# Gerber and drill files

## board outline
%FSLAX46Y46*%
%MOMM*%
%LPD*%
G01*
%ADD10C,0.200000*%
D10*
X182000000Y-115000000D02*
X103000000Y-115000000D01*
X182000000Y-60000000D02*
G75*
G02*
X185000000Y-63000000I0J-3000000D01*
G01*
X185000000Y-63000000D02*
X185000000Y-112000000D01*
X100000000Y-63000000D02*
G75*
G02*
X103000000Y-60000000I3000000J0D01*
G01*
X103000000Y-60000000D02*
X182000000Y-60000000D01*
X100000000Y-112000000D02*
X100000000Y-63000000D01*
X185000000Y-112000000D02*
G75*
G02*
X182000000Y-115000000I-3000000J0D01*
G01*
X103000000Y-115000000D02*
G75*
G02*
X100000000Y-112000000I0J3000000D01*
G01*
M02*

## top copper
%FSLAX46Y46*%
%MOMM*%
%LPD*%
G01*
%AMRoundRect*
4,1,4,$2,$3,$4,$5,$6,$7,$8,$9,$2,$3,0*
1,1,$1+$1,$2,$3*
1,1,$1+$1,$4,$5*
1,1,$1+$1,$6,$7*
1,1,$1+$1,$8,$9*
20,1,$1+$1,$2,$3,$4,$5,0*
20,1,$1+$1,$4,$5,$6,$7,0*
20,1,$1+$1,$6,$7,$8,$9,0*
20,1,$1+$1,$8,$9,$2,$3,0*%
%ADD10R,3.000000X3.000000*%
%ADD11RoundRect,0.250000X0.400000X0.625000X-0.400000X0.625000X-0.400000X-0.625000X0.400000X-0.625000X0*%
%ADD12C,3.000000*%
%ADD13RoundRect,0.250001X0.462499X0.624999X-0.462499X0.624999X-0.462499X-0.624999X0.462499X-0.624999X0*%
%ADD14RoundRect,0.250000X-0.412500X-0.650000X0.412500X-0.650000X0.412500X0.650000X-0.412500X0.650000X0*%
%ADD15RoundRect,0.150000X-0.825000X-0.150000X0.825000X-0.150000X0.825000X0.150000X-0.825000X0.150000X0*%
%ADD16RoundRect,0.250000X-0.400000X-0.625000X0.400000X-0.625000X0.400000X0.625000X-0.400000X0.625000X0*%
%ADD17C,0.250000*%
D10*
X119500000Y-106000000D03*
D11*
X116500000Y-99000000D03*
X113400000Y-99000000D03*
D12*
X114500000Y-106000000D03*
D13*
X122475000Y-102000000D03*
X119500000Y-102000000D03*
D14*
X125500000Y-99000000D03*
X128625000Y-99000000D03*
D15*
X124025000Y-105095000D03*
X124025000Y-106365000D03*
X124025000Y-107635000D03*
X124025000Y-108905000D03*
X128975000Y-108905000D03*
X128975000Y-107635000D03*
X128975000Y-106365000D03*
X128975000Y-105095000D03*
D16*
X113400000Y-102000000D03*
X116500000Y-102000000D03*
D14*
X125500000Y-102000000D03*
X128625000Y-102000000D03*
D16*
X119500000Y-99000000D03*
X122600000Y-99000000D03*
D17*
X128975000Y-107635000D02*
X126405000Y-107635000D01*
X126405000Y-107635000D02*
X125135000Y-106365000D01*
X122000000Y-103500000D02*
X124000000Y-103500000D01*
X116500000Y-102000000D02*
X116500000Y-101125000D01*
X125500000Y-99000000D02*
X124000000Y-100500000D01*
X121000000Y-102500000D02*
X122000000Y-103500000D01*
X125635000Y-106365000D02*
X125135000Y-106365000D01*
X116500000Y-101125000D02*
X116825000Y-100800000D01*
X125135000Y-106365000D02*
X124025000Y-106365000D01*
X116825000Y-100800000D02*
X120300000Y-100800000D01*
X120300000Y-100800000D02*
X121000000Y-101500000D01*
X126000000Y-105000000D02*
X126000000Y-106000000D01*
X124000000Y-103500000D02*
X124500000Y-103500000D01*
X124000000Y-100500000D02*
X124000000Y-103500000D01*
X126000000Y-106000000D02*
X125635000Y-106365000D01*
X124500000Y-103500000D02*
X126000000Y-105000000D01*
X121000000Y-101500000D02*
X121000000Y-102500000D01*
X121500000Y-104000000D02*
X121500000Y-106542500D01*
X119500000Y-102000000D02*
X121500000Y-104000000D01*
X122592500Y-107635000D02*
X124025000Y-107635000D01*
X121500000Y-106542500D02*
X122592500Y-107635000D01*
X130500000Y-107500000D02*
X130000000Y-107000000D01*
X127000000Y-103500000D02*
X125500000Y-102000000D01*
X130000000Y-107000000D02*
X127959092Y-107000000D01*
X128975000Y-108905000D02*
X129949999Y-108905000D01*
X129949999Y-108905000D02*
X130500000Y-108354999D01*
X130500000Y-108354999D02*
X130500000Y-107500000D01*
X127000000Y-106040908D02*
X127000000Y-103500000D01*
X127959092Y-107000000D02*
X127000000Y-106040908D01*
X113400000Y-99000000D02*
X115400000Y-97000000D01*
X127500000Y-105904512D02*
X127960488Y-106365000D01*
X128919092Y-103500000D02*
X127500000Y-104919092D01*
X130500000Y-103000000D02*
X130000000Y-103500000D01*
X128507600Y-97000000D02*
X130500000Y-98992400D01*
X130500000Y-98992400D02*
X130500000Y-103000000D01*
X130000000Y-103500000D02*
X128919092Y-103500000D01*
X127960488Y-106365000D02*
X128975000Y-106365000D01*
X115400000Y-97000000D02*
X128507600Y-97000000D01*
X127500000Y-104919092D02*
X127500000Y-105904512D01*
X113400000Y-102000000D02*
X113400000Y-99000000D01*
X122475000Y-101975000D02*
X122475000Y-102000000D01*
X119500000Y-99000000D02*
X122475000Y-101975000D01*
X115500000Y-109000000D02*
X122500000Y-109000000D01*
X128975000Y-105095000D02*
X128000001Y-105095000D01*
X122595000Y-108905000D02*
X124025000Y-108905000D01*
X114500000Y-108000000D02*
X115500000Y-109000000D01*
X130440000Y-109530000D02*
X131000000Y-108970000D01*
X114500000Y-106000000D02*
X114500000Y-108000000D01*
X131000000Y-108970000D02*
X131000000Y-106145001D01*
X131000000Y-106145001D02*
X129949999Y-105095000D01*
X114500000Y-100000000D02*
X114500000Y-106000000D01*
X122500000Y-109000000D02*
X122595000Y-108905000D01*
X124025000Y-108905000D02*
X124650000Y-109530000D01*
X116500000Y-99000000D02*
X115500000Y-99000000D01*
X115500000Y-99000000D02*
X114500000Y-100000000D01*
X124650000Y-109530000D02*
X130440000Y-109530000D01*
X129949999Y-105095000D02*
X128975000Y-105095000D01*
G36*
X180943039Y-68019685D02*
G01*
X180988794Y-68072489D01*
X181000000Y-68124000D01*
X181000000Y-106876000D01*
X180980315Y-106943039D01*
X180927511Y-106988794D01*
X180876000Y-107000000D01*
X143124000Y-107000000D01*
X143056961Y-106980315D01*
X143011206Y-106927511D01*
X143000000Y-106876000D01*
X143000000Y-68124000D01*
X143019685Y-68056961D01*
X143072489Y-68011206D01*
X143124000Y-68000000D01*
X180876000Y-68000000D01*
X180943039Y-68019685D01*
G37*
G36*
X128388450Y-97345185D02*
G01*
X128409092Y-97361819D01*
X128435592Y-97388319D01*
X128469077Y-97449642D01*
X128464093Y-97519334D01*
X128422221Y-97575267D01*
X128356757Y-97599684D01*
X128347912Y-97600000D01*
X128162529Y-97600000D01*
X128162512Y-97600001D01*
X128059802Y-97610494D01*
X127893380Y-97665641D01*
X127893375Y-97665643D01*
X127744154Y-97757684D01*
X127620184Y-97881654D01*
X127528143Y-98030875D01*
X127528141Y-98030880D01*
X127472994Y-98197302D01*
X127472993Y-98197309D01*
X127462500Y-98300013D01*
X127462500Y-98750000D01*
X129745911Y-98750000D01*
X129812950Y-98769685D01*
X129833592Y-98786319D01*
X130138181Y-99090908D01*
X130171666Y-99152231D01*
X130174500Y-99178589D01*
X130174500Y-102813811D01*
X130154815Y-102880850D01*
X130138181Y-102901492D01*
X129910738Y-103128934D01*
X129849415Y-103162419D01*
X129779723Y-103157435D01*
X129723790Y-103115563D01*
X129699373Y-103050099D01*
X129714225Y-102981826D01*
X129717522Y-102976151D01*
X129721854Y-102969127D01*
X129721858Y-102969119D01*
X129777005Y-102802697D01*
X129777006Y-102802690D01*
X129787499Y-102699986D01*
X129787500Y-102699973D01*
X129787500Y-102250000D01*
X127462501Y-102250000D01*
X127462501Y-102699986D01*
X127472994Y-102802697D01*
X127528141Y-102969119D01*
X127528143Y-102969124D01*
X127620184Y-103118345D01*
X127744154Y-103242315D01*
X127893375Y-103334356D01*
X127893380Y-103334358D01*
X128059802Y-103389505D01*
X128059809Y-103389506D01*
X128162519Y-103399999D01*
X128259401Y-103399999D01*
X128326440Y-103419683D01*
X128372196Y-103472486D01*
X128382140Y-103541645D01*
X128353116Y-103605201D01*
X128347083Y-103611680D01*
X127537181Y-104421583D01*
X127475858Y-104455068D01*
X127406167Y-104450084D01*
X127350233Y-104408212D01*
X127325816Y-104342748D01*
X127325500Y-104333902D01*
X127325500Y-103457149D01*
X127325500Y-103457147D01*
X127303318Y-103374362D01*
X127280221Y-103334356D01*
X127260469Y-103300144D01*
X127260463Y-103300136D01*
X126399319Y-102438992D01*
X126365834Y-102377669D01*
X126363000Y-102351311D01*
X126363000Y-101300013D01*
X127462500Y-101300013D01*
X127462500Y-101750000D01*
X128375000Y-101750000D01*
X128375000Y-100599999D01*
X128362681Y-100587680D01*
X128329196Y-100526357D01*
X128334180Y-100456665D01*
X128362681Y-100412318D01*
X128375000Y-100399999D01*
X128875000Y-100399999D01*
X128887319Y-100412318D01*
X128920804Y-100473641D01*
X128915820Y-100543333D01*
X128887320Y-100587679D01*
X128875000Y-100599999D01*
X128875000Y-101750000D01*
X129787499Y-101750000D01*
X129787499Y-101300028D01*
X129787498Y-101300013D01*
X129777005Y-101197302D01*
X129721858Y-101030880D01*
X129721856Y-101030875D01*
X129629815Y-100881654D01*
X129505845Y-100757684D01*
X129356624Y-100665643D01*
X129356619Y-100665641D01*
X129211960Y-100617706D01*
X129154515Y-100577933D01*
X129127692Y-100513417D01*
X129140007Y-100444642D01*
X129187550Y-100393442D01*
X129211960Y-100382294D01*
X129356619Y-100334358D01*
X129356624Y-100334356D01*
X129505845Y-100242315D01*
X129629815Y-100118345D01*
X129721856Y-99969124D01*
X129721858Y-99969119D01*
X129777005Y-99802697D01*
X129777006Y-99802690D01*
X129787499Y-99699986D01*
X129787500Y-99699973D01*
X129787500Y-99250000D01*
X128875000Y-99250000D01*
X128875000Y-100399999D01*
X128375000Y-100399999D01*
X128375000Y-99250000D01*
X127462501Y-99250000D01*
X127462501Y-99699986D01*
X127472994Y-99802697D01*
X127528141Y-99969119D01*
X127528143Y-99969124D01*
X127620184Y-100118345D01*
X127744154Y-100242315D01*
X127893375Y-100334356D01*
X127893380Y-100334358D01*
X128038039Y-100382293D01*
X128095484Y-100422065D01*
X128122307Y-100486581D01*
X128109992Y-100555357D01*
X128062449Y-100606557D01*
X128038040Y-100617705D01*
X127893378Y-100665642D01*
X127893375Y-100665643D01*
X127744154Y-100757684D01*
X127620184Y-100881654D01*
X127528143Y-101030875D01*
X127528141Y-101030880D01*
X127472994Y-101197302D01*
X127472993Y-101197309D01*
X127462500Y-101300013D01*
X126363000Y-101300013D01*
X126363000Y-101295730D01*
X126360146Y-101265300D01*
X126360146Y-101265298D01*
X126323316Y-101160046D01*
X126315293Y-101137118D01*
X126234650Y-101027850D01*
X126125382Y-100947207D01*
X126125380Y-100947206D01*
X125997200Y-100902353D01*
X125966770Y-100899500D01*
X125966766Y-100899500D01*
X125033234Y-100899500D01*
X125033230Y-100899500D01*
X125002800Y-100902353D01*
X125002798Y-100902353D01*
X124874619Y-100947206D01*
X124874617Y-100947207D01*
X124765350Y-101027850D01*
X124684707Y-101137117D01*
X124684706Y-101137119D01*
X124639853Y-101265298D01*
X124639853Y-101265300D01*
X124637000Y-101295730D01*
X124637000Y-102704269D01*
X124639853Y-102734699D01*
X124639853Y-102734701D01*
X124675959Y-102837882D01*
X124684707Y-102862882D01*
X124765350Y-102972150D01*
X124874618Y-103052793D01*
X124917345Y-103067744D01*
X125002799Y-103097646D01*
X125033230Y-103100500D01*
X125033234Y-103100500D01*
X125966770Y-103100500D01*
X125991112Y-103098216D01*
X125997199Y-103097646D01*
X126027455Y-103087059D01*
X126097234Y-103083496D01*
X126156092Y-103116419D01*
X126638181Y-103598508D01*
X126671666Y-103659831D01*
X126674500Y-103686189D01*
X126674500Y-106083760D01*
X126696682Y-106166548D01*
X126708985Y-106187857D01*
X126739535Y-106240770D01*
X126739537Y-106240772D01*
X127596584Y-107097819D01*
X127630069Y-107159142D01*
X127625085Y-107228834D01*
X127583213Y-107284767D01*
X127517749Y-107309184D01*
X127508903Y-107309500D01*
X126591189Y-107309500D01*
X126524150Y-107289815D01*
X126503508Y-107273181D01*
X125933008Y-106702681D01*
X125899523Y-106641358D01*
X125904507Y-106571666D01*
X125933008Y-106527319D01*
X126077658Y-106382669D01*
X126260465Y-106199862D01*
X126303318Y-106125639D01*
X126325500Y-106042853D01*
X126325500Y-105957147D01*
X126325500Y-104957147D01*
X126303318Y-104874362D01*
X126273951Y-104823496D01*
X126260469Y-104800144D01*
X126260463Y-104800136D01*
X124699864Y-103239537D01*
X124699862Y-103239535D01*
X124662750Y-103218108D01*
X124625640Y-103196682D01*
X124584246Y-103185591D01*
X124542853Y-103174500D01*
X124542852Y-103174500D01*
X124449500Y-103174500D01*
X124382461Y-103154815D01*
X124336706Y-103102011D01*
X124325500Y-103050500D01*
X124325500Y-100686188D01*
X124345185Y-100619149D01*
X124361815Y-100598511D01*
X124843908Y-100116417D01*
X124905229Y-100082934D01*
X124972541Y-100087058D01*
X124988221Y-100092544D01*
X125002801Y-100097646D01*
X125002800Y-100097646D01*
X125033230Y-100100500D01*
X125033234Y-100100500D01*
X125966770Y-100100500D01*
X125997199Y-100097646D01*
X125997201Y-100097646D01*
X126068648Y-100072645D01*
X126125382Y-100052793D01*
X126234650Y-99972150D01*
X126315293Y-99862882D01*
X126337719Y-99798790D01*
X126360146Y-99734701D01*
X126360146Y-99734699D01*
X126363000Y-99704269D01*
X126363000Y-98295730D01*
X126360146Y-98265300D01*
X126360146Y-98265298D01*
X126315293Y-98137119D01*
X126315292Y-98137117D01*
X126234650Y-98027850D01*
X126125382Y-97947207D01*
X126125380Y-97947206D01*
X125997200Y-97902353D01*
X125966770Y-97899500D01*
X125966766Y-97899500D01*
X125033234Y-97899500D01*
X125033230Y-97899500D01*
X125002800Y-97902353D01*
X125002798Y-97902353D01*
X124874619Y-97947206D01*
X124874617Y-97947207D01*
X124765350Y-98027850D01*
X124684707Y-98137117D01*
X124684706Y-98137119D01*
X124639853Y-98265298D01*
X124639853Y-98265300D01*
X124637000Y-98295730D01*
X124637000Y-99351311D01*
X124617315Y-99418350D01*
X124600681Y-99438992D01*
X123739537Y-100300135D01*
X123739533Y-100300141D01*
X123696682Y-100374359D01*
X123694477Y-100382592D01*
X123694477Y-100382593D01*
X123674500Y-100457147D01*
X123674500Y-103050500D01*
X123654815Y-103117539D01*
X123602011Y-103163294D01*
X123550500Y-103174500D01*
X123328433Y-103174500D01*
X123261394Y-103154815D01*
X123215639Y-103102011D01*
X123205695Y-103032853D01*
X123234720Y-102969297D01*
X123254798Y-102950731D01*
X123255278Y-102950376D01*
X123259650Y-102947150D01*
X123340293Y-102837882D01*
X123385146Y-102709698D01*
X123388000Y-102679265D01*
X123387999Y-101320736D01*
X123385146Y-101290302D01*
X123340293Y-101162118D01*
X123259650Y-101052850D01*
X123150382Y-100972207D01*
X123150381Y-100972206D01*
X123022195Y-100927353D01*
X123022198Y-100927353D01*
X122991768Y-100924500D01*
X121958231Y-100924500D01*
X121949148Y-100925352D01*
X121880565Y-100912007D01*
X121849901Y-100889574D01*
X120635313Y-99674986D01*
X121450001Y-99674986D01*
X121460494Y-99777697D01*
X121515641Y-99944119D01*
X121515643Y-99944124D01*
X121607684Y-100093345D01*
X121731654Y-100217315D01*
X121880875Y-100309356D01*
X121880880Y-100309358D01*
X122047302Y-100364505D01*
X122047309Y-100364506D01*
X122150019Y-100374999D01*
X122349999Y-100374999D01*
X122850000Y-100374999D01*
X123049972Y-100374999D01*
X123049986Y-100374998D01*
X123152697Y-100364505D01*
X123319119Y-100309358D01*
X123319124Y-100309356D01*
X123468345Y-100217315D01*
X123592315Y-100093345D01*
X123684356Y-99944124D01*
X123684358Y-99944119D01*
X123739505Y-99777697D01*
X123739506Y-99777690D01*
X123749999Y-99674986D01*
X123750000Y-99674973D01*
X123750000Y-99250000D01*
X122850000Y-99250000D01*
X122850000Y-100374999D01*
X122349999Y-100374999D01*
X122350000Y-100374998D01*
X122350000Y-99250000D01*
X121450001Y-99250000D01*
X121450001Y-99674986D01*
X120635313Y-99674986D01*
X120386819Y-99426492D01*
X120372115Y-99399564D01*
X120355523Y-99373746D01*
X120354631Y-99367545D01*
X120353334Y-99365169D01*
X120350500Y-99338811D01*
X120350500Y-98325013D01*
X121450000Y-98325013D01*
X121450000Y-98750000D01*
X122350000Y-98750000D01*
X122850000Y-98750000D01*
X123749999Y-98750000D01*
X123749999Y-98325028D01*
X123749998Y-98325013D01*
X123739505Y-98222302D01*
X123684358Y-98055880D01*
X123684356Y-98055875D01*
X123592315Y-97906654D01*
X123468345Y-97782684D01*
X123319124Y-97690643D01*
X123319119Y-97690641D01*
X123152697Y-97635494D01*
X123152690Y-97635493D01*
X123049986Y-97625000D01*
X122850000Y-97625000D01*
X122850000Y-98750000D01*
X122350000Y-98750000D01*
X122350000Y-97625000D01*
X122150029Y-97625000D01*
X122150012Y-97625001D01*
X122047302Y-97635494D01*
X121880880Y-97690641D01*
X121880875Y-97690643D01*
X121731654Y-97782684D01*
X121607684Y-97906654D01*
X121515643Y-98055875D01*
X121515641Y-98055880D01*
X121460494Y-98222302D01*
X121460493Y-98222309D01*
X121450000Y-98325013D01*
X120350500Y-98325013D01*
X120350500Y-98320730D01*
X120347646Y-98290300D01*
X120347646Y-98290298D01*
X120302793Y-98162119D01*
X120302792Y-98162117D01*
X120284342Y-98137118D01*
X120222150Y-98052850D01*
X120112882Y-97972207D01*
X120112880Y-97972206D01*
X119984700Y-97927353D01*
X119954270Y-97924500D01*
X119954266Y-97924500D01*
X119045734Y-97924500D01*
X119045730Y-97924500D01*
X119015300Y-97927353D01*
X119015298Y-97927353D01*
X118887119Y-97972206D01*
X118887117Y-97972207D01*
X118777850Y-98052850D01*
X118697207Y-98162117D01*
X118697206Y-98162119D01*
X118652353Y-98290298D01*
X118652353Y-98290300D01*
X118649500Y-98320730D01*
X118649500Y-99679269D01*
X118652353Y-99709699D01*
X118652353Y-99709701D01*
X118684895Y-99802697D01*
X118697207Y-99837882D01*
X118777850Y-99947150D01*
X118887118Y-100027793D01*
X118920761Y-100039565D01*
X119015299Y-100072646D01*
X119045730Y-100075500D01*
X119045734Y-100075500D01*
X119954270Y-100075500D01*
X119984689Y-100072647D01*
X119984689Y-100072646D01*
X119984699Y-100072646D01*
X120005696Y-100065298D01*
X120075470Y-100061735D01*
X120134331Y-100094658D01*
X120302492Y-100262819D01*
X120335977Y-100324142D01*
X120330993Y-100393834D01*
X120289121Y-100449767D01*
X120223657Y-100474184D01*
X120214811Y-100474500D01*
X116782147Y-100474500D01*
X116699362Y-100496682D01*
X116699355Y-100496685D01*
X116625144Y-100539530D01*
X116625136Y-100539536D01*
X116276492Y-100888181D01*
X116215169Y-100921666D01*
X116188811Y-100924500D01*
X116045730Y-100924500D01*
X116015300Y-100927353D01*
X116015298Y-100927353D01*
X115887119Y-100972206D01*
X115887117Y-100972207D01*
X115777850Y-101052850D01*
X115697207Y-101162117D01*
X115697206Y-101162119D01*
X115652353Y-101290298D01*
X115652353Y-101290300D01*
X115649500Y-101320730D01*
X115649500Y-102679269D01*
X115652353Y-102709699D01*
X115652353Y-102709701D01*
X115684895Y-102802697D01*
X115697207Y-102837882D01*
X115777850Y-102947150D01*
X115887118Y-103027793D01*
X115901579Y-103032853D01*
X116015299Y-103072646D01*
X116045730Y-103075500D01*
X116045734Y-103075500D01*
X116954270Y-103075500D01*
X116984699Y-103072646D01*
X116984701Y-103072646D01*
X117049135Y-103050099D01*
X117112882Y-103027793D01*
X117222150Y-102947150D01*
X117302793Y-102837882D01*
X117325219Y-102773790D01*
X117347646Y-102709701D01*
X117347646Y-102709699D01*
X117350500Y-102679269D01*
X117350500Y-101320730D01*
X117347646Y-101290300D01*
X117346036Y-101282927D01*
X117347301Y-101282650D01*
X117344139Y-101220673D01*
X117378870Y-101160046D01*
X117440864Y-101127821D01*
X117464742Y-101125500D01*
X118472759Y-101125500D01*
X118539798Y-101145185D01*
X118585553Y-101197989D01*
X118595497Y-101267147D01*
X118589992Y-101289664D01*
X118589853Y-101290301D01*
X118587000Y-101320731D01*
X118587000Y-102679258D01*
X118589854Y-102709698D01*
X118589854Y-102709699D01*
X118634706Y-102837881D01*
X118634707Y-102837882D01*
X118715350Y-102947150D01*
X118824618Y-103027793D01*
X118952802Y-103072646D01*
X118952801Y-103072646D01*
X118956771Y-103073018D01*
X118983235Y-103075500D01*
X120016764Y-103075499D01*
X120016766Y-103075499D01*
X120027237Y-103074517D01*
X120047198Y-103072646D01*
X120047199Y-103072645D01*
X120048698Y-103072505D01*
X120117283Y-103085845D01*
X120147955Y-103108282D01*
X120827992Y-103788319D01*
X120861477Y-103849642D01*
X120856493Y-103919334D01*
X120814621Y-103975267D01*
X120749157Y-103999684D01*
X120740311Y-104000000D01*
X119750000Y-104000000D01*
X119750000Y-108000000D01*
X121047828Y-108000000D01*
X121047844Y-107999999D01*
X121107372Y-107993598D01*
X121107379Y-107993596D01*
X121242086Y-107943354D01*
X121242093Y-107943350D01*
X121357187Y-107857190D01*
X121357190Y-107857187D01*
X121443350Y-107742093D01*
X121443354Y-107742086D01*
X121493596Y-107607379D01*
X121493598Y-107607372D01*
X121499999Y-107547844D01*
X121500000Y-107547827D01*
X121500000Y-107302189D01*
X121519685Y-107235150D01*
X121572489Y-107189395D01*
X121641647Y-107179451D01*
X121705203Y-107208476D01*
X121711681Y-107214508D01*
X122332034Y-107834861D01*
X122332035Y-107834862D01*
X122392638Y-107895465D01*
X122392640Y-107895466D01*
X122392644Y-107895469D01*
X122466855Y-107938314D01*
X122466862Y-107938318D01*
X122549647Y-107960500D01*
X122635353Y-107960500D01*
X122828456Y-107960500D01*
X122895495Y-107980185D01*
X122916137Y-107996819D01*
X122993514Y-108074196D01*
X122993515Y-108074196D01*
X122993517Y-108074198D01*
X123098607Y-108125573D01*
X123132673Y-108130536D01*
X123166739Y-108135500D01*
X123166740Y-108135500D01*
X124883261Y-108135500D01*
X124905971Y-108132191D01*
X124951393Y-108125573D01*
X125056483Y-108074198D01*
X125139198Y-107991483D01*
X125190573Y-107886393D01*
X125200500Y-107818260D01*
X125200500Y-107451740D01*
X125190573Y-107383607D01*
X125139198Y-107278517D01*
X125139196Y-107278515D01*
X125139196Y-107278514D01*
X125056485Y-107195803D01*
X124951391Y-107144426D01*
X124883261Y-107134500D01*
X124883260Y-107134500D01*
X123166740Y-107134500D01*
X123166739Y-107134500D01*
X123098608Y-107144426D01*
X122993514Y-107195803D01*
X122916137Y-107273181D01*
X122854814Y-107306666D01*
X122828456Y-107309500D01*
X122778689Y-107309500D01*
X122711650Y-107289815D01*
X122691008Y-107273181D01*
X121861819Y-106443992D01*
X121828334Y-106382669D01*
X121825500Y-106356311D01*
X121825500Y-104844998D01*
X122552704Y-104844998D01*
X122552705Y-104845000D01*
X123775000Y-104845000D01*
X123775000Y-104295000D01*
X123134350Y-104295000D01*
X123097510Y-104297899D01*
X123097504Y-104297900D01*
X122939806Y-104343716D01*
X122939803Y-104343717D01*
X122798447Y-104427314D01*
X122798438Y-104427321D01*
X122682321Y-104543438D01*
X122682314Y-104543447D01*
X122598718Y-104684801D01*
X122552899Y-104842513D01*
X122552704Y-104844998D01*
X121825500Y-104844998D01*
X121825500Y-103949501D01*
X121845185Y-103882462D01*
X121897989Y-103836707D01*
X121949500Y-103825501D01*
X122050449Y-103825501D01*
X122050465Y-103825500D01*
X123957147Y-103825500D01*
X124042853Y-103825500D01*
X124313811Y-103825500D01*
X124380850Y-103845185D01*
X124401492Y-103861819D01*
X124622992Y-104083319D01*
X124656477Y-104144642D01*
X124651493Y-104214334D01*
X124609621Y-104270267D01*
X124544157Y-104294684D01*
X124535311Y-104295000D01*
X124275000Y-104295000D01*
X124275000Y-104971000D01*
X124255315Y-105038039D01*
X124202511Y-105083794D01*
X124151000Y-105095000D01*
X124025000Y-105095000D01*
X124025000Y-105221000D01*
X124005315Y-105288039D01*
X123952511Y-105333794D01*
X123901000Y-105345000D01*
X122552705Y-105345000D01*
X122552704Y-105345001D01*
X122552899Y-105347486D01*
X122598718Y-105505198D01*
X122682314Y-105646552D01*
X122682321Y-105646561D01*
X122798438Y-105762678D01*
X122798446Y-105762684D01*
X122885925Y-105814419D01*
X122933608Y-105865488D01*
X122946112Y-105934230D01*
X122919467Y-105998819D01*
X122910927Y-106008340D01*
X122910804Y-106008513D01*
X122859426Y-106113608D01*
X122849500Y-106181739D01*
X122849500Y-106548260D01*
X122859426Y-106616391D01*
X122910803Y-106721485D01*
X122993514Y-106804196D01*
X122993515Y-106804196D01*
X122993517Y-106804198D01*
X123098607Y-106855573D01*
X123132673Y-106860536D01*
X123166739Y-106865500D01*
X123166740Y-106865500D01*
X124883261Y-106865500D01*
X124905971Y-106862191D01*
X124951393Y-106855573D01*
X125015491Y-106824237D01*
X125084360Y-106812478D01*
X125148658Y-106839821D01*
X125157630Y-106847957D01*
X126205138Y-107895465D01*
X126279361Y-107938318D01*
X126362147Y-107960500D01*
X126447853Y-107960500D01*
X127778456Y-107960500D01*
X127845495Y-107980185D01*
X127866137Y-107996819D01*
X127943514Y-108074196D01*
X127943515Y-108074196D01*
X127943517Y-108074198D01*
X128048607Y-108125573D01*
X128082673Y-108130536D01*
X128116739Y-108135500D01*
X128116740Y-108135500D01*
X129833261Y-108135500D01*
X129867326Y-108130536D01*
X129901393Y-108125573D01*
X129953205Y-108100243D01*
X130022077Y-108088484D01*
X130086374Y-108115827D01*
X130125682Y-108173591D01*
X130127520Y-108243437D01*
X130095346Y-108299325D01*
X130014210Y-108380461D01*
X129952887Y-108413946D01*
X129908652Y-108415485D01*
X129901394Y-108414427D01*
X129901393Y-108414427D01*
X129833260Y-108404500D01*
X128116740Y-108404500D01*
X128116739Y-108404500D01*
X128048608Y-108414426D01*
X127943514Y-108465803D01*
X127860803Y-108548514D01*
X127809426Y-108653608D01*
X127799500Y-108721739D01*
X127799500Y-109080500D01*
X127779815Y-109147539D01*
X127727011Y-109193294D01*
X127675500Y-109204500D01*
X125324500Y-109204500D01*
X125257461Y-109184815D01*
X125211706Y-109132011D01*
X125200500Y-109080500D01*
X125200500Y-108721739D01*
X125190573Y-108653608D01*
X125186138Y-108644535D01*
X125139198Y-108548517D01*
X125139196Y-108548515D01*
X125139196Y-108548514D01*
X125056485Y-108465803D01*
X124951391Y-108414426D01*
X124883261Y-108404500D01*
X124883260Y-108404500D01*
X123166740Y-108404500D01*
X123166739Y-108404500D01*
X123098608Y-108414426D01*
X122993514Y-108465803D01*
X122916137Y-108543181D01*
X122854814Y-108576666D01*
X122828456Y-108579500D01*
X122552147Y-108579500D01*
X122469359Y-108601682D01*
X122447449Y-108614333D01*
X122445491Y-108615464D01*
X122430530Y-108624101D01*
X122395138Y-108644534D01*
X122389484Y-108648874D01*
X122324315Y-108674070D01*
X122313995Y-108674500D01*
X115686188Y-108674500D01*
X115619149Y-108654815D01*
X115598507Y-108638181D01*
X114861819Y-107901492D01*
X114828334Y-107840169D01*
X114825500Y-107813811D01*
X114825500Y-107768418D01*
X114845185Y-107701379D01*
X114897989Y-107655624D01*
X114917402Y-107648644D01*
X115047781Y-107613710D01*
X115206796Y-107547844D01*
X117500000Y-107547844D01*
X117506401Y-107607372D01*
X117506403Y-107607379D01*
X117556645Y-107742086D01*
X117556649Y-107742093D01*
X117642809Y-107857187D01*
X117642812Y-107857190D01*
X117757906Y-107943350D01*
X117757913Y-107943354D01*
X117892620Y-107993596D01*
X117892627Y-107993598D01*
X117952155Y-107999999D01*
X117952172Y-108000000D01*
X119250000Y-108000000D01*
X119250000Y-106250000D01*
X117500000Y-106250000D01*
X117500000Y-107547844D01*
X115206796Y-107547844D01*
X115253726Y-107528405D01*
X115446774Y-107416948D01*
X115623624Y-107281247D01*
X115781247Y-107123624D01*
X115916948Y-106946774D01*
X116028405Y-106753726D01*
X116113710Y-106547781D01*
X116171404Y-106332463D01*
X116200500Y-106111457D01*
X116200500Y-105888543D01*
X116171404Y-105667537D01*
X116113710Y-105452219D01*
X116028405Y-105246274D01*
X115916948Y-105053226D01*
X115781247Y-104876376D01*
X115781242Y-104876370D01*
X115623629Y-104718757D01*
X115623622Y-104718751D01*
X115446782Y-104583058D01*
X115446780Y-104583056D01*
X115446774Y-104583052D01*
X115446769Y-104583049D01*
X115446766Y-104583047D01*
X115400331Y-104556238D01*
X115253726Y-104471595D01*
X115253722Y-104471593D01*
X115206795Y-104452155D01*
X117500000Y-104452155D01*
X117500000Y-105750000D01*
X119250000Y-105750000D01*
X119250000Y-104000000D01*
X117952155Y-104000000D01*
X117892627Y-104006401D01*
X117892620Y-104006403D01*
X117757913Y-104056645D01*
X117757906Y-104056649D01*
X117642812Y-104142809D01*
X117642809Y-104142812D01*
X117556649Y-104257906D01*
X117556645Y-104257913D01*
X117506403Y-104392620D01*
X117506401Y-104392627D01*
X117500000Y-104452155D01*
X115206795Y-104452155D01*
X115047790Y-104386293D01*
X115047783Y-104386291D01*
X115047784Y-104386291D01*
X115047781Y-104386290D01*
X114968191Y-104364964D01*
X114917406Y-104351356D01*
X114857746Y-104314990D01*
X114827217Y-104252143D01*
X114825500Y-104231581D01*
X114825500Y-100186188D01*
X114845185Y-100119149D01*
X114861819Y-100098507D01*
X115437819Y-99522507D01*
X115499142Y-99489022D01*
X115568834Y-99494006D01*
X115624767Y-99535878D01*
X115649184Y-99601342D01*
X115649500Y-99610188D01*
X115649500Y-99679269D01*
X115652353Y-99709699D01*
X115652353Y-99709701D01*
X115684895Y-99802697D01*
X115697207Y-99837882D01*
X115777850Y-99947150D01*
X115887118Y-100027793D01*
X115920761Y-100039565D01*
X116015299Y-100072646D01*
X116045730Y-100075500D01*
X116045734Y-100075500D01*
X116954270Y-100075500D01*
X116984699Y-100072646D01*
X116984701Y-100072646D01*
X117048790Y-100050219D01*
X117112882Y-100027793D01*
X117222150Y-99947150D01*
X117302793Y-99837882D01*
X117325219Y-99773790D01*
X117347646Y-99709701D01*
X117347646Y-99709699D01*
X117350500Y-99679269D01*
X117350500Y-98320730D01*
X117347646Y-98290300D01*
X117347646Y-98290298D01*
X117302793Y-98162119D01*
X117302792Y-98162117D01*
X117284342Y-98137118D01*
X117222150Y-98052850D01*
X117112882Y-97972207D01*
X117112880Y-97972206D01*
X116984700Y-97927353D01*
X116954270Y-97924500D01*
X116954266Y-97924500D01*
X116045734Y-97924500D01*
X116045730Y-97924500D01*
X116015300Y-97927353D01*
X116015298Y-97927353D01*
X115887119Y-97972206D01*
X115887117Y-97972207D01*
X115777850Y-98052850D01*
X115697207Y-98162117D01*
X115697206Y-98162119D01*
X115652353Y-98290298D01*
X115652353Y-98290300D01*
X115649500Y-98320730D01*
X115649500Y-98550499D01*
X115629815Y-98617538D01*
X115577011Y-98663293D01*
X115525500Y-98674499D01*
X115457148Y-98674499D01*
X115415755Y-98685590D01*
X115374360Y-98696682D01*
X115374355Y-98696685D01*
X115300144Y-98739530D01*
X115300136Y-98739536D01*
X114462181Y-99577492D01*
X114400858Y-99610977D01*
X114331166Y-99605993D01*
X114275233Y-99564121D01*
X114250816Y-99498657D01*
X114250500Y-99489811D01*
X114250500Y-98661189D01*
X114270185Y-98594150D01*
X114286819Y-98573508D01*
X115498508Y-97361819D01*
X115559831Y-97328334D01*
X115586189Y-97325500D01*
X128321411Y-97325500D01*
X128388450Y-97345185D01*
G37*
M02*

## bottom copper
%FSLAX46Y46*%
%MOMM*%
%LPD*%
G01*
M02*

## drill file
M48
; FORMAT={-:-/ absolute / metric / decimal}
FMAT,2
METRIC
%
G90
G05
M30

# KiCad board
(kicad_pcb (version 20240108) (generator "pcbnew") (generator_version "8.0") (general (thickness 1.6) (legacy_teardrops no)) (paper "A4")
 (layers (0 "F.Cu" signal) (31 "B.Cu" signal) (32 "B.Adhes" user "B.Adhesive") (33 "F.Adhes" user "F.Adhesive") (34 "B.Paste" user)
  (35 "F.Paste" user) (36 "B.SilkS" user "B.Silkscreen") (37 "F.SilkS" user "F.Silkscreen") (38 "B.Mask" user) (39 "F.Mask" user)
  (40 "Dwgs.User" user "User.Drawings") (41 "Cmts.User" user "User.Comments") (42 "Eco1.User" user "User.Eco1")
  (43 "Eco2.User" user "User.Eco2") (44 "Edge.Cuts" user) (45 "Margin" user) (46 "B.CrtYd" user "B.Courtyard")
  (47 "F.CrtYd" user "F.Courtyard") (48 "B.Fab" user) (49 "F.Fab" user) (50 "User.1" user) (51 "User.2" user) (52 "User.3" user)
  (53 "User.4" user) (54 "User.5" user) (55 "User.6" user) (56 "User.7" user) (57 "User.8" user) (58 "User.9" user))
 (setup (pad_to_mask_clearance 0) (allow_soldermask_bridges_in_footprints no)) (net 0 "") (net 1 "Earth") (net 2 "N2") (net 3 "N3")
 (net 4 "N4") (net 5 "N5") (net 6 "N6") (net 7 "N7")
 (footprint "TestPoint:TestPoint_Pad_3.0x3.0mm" (layer "F.Cu") (at 119.5 106)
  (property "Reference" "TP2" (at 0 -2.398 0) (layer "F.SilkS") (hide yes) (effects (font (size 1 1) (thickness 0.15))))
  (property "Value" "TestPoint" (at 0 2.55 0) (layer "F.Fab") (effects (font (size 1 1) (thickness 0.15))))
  (pad "1" smd rect (at 0 0) (size 3 3) (layers "F.Cu" "F.Mask") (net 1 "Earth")))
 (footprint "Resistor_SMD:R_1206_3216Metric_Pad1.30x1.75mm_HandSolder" (layer "F.Cu") (at 114.95 99 180)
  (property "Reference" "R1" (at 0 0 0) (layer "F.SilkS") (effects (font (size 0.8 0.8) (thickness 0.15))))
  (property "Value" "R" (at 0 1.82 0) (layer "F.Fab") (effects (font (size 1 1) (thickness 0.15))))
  (pad "1" smd roundrect (at -1.55 0 180) (size 1.3 1.75) (layers "F.Cu" "F.Paste" "F.Mask") (roundrect_rratio 0.1923076923) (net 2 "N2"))
  (pad "2" smd roundrect (at 1.55 0 180) (size 1.3 1.75) (layers "F.Cu" "F.Paste" "F.Mask") (roundrect_rratio 0.1923076923) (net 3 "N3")))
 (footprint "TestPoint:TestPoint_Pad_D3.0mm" (layer "F.Cu") (at 114.5 106)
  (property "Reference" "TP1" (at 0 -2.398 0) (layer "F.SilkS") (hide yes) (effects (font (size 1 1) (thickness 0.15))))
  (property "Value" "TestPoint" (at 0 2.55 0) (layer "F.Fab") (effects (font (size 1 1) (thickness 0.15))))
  (pad "1" smd circle (at 0 0) (size 3 3) (layers "F.Cu" "F.Mask") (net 2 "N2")))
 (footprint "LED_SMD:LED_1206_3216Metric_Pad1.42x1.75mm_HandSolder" (layer "F.Cu") (at 120.9875 102 180)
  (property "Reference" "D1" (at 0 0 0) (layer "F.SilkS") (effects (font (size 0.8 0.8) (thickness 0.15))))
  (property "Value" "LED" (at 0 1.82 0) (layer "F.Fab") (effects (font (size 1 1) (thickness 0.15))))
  (pad "1" smd roundrect (at -1.4875 0 180) (size 1.425 1.75) (layers "F.Cu" "F.Paste" "F.Mask") (roundrect_rratio 0.1754392982)
   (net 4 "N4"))
  (pad "2" smd roundrect (at 1.4875 0 180) (size 1.425 1.75) (layers "F.Cu" "F.Paste" "F.Mask") (roundrect_rratio 0.1754392982) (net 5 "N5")))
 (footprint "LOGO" (layer "F.Cu") (at 162 87.5)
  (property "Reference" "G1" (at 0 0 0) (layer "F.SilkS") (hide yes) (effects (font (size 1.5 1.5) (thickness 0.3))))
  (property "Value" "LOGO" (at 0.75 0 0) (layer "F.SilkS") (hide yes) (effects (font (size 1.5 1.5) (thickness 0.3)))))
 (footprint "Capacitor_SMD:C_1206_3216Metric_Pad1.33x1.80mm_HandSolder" (layer "F.Cu") (at 127.0625 99)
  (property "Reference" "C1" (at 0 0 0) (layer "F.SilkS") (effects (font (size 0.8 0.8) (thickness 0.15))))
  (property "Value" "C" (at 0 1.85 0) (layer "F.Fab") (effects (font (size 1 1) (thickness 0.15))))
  (pad "1" smd roundrect (at -1.5625 0) (size 1.325 1.8) (layers "F.Cu" "F.Paste" "F.Mask") (roundrect_rratio 0.1886792453) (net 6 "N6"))
  (pad "2" smd roundrect (at 1.5625 0) (size 1.325 1.8) (layers "F.Cu" "F.Paste" "F.Mask") (roundrect_rratio 0.1886792453) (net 1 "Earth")))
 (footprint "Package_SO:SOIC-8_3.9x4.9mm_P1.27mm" (layer "F.Cu") (at 126.5 107)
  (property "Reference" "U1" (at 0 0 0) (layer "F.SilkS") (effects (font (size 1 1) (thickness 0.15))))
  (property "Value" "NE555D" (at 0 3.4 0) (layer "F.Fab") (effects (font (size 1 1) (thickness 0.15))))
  (pad "1" smd roundrect (at -2.475 -1.905) (size 1.95 0.6) (layers "F.Cu" "F.Paste" "F.Mask") (roundrect_rratio 0.25) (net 1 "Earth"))
  (pad "2" smd roundrect (at -2.475 -0.635) (size 1.95 0.6) (layers "F.Cu" "F.Paste" "F.Mask") (roundrect_rratio 0.25) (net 6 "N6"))
  (pad "3" smd roundrect (at -2.475 0.635) (size 1.95 0.6) (layers "F.Cu" "F.Paste" "F.Mask") (roundrect_rratio 0.25) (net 5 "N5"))
  (pad "4" smd roundrect (at -2.475 1.905) (size 1.95 0.6) (layers "F.Cu" "F.Paste" "F.Mask") (roundrect_rratio 0.25) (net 2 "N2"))
  (pad "5" smd roundrect (at 2.475 1.905) (size 1.95 0.6) (layers "F.Cu" "F.Paste" "F.Mask") (roundrect_rratio 0.25) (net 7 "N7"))
  (pad "6" smd roundrect (at 2.475 0.635) (size 1.95 0.6) (layers "F.Cu" "F.Paste" "F.Mask") (roundrect_rratio 0.25) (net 6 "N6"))
  (pad "7" smd roundrect (at 2.475 -0.635) (size 1.95 0.6) (layers "F.Cu" "F.Paste" "F.Mask") (roundrect_rratio 0.25) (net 3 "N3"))
  (pad "8" smd roundrect (at 2.475 -1.905) (size 1.95 0.6) (layers "F.Cu" "F.Paste" "F.Mask") (roundrect_rratio 0.25) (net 2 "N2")))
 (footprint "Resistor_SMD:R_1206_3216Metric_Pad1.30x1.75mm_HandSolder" (layer "F.Cu") (at 114.95 102)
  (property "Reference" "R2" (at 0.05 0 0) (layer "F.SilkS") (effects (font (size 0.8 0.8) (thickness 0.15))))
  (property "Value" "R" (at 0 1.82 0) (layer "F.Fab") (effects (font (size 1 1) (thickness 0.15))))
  (pad "1" smd roundrect (at -1.55 0) (size 1.3 1.75) (layers "F.Cu" "F.Paste" "F.Mask") (roundrect_rratio 0.1923076923) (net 3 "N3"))
  (pad "2" smd roundrect (at 1.55 0) (size 1.3 1.75) (layers "F.Cu" "F.Paste" "F.Mask") (roundrect_rratio 0.1923076923) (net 6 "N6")))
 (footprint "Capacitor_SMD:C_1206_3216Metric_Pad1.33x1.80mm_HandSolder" (layer "F.Cu") (at 127.0625 102)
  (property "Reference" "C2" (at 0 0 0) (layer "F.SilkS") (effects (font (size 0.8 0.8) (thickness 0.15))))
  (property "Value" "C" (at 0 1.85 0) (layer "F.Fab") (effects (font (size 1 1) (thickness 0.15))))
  (pad "1" smd roundrect (at -1.5625 0) (size 1.325 1.8) (layers "F.Cu" "F.Paste" "F.Mask") (roundrect_rratio 0.1886792453) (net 7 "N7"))
  (pad "2" smd roundrect (at 1.5625 0) (size 1.325 1.8) (layers "F.Cu" "F.Paste" "F.Mask") (roundrect_rratio 0.1886792453) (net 1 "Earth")))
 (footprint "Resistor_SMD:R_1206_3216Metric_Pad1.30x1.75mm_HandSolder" (layer "F.Cu") (at 121.05 99)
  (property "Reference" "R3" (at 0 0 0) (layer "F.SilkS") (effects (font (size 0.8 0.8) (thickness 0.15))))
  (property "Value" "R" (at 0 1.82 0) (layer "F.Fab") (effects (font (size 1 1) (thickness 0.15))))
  (pad "1" smd roundrect (at -1.55 0) (size 1.3 1.75) (layers "F.Cu" "F.Paste" "F.Mask") (roundrect_rratio 0.1923076923) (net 4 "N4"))
  (pad "2" smd roundrect (at 1.55 0) (size 1.3 1.75) (layers "F.Cu" "F.Paste" "F.Mask") (roundrect_rratio 0.1923076923) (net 1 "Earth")))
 (gr_line (start 182 115) (end 103 115) (stroke (width 0.2) (type default)) (layer "Edge.Cuts"))
 (gr_arc (start 182 60) (mid 184.121321 60.878679) (end 185 63) (stroke (width 0.2) (type default)) (layer "Edge.Cuts"))
 (gr_line (start 185 63) (end 185 112) (stroke (width 0.2) (type default)) (layer "Edge.Cuts"))
 (gr_arc (start 100 63) (mid 100.878679 60.878679) (end 103 60) (stroke (width 0.2) (type default)) (layer "Edge.Cuts"))
 (gr_line (start 103 60) (end 182 60) (stroke (width 0.2) (type default)) (layer "Edge.Cuts"))
 (gr_line (start 100 112) (end 100 63) (stroke (width 0.2) (type default)) (layer "Edge.Cuts"))
 (gr_arc (start 185 112) (mid 184.121321 114.121321) (end 182 115) (stroke (width 0.2) (type default)) (layer "Edge.Cuts"))
 (gr_arc (start 103 115) (mid 100.878679 114.121321) (end 100 112) (stroke (width 0.2) (type default)) (layer "Edge.Cuts"))
 (segment (start 128.975 107.635) (end 126.405 107.635) (width 0.25) (layer "F.Cu") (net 6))
 (segment (start 126.405 107.635) (end 125.135 106.365) (width 0.25) (layer "F.Cu") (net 6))
 (segment (start 122 103.5) (end 124 103.5) (width 0.25) (layer "F.Cu") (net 6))
 (segment (start 116.5 102) (end 116.5 101.125) (width 0.25) (layer "F.Cu") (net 6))
 (segment (start 125.5 99) (end 124 100.5) (width 0.25) (layer "F.Cu") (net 6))
 (segment (start 121 102.5) (end 122 103.5) (width 0.25) (layer "F.Cu") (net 6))
 (segment (start 125.635 106.365) (end 125.135 106.365) (width 0.25) (layer "F.Cu") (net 6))
 (segment (start 116.5 101.125) (end 116.825 100.8) (width 0.25) (layer "F.Cu") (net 6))
 (segment (start 125.135 106.365) (end 124.025 106.365) (width 0.25) (layer "F.Cu") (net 6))
 (segment (start 116.825 100.8) (end 120.3 100.8) (width 0.25) (layer "F.Cu") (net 6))
 (segment (start 120.3 100.8) (end 121 101.5) (width 0.25) (layer "F.Cu") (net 6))
 (segment (start 126 105) (end 126 106) (width 0.25) (layer "F.Cu") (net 6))
 (segment (start 124 103.5) (end 124.5 103.5) (width 0.25) (layer "F.Cu") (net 6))
 (segment (start 124 100.5) (end 124 103.5) (width 0.25) (layer "F.Cu") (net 6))
 (segment (start 126 106) (end 125.635 106.365) (width 0.25) (layer "F.Cu") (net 6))
 (segment (start 124.5 103.5) (end 126 105) (width 0.25) (layer "F.Cu") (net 6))
 (segment (start 121 101.5) (end 121 102.5) (width 0.25) (layer "F.Cu") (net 6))
 (segment (start 121.5 104) (end 121.5 106.5425) (width 0.25) (layer "F.Cu") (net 5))
 (segment (start 119.5 102) (end 121.5 104) (width 0.25) (layer "F.Cu") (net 5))
 (segment (start 122.5925 107.635) (end 124.025 107.635) (width 0.25) (layer "F.Cu") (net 5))
 (segment (start 121.5 106.5425) (end 122.5925 107.635) (width 0.25) (layer "F.Cu") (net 5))
 (segment (start 130.5 107.5) (end 130 107) (width 0.25) (layer "F.Cu") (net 7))
 (segment (start 127 103.5) (end 125.5 102) (width 0.25) (layer "F.Cu") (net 7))
 (segment (start 130 107) (end 127.959092 107) (width 0.25) (layer "F.Cu") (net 7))
 (segment (start 128.975 108.905) (end 129.949999 108.905) (width 0.25) (layer "F.Cu") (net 7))
 (segment (start 129.949999 108.905) (end 130.5 108.354999) (width 0.25) (layer "F.Cu") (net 7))
 (segment (start 130.5 108.354999) (end 130.5 107.5) (width 0.25) (layer "F.Cu") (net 7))
 (segment (start 127 106.040908) (end 127 103.5) (width 0.25) (layer "F.Cu") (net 7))
 (segment (start 127.959092 107) (end 127 106.040908) (width 0.25) (layer "F.Cu") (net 7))
 (segment (start 113.4 99) (end 115.4 97) (width 0.25) (layer "F.Cu") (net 3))
 (segment (start 127.5 105.904512) (end 127.960488 106.365) (width 0.25) (layer "F.Cu") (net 3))
 (segment (start 128.919092 103.5) (end 127.5 104.919092) (width 0.25) (layer "F.Cu") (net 3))
 (segment (start 130.5 103) (end 130 103.5) (width 0.25) (layer "F.Cu") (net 3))
 (segment (start 128.5076 97) (end 130.5 98.9924) (width 0.25) (layer "F.Cu") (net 3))
 (segment (start 130.5 98.9924) (end 130.5 103) (width 0.25) (layer "F.Cu") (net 3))
 (segment (start 130 103.5) (end 128.919092 103.5) (width 0.25) (layer "F.Cu") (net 3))
 (segment (start 127.960488 106.365) (end 128.975 106.365) (width 0.25) (layer "F.Cu") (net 3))
 (segment (start 115.4 97) (end 128.5076 97) (width 0.25) (layer "F.Cu") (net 3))
 (segment (start 127.5 104.919092) (end 127.5 105.904512) (width 0.25) (layer "F.Cu") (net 3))
 (segment (start 113.4 102) (end 113.4 99) (width 0.25) (layer "F.Cu") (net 3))
 (segment (start 122.475 101.975) (end 122.475 102) (width 0.25) (layer "F.Cu") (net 4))
 (segment (start 119.5 99) (end 122.475 101.975) (width 0.25) (layer "F.Cu") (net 4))
 (segment (start 115.5 109) (end 122.5 109) (width 0.25) (layer "F.Cu") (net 2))
 (segment (start 128.975 105.095) (end 128.000001 105.095) (width 0.25) (layer "F.Cu") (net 2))
 (segment (start 122.595 108.905) (end 124.025 108.905) (width 0.25) (layer "F.Cu") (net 2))
 (segment (start 114.5 108) (end 115.5 109) (width 0.25) (layer "F.Cu") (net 2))
 (segment (start 130.44 109.53) (end 131 108.97) (width 0.25) (layer "F.Cu") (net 2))
 (segment (start 114.5 106) (end 114.5 108) (width 0.25) (layer "F.Cu") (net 2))
 (segment (start 131 108.97) (end 131 106.145001) (width 0.25) (layer "F.Cu") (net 2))
 (segment (start 131 106.145001) (end 129.949999 105.095) (width 0.25) (layer "F.Cu") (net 2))
 (segment (start 114.5 100) (end 114.5 106) (width 0.25) (layer "F.Cu") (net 2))
 (segment (start 122.5 109) (end 122.595 108.905) (width 0.25) (layer "F.Cu") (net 2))
 (segment (start 124.025 108.905) (end 124.65 109.53) (width 0.25) (layer "F.Cu") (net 2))
 (segment (start 116.5 99) (end 115.5 99) (width 0.25) (layer "F.Cu") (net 2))
 (segment (start 115.5 99) (end 114.5 100) (width 0.25) (layer "F.Cu") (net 2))
 (segment (start 124.65 109.53) (end 130.44 109.53) (width 0.25) (layer "F.Cu") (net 2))
 (segment (start 129.949999 105.095) (end 128.975 105.095) (width 0.25) (layer "F.Cu") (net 2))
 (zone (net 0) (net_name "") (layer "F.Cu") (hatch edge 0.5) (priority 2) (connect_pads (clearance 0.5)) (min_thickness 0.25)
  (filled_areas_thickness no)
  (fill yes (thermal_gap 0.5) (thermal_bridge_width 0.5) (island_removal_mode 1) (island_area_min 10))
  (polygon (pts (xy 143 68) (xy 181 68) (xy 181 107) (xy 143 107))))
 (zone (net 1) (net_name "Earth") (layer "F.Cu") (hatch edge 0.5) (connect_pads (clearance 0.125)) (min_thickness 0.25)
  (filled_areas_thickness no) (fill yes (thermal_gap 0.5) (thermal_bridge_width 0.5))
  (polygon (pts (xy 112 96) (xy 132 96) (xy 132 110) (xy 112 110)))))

